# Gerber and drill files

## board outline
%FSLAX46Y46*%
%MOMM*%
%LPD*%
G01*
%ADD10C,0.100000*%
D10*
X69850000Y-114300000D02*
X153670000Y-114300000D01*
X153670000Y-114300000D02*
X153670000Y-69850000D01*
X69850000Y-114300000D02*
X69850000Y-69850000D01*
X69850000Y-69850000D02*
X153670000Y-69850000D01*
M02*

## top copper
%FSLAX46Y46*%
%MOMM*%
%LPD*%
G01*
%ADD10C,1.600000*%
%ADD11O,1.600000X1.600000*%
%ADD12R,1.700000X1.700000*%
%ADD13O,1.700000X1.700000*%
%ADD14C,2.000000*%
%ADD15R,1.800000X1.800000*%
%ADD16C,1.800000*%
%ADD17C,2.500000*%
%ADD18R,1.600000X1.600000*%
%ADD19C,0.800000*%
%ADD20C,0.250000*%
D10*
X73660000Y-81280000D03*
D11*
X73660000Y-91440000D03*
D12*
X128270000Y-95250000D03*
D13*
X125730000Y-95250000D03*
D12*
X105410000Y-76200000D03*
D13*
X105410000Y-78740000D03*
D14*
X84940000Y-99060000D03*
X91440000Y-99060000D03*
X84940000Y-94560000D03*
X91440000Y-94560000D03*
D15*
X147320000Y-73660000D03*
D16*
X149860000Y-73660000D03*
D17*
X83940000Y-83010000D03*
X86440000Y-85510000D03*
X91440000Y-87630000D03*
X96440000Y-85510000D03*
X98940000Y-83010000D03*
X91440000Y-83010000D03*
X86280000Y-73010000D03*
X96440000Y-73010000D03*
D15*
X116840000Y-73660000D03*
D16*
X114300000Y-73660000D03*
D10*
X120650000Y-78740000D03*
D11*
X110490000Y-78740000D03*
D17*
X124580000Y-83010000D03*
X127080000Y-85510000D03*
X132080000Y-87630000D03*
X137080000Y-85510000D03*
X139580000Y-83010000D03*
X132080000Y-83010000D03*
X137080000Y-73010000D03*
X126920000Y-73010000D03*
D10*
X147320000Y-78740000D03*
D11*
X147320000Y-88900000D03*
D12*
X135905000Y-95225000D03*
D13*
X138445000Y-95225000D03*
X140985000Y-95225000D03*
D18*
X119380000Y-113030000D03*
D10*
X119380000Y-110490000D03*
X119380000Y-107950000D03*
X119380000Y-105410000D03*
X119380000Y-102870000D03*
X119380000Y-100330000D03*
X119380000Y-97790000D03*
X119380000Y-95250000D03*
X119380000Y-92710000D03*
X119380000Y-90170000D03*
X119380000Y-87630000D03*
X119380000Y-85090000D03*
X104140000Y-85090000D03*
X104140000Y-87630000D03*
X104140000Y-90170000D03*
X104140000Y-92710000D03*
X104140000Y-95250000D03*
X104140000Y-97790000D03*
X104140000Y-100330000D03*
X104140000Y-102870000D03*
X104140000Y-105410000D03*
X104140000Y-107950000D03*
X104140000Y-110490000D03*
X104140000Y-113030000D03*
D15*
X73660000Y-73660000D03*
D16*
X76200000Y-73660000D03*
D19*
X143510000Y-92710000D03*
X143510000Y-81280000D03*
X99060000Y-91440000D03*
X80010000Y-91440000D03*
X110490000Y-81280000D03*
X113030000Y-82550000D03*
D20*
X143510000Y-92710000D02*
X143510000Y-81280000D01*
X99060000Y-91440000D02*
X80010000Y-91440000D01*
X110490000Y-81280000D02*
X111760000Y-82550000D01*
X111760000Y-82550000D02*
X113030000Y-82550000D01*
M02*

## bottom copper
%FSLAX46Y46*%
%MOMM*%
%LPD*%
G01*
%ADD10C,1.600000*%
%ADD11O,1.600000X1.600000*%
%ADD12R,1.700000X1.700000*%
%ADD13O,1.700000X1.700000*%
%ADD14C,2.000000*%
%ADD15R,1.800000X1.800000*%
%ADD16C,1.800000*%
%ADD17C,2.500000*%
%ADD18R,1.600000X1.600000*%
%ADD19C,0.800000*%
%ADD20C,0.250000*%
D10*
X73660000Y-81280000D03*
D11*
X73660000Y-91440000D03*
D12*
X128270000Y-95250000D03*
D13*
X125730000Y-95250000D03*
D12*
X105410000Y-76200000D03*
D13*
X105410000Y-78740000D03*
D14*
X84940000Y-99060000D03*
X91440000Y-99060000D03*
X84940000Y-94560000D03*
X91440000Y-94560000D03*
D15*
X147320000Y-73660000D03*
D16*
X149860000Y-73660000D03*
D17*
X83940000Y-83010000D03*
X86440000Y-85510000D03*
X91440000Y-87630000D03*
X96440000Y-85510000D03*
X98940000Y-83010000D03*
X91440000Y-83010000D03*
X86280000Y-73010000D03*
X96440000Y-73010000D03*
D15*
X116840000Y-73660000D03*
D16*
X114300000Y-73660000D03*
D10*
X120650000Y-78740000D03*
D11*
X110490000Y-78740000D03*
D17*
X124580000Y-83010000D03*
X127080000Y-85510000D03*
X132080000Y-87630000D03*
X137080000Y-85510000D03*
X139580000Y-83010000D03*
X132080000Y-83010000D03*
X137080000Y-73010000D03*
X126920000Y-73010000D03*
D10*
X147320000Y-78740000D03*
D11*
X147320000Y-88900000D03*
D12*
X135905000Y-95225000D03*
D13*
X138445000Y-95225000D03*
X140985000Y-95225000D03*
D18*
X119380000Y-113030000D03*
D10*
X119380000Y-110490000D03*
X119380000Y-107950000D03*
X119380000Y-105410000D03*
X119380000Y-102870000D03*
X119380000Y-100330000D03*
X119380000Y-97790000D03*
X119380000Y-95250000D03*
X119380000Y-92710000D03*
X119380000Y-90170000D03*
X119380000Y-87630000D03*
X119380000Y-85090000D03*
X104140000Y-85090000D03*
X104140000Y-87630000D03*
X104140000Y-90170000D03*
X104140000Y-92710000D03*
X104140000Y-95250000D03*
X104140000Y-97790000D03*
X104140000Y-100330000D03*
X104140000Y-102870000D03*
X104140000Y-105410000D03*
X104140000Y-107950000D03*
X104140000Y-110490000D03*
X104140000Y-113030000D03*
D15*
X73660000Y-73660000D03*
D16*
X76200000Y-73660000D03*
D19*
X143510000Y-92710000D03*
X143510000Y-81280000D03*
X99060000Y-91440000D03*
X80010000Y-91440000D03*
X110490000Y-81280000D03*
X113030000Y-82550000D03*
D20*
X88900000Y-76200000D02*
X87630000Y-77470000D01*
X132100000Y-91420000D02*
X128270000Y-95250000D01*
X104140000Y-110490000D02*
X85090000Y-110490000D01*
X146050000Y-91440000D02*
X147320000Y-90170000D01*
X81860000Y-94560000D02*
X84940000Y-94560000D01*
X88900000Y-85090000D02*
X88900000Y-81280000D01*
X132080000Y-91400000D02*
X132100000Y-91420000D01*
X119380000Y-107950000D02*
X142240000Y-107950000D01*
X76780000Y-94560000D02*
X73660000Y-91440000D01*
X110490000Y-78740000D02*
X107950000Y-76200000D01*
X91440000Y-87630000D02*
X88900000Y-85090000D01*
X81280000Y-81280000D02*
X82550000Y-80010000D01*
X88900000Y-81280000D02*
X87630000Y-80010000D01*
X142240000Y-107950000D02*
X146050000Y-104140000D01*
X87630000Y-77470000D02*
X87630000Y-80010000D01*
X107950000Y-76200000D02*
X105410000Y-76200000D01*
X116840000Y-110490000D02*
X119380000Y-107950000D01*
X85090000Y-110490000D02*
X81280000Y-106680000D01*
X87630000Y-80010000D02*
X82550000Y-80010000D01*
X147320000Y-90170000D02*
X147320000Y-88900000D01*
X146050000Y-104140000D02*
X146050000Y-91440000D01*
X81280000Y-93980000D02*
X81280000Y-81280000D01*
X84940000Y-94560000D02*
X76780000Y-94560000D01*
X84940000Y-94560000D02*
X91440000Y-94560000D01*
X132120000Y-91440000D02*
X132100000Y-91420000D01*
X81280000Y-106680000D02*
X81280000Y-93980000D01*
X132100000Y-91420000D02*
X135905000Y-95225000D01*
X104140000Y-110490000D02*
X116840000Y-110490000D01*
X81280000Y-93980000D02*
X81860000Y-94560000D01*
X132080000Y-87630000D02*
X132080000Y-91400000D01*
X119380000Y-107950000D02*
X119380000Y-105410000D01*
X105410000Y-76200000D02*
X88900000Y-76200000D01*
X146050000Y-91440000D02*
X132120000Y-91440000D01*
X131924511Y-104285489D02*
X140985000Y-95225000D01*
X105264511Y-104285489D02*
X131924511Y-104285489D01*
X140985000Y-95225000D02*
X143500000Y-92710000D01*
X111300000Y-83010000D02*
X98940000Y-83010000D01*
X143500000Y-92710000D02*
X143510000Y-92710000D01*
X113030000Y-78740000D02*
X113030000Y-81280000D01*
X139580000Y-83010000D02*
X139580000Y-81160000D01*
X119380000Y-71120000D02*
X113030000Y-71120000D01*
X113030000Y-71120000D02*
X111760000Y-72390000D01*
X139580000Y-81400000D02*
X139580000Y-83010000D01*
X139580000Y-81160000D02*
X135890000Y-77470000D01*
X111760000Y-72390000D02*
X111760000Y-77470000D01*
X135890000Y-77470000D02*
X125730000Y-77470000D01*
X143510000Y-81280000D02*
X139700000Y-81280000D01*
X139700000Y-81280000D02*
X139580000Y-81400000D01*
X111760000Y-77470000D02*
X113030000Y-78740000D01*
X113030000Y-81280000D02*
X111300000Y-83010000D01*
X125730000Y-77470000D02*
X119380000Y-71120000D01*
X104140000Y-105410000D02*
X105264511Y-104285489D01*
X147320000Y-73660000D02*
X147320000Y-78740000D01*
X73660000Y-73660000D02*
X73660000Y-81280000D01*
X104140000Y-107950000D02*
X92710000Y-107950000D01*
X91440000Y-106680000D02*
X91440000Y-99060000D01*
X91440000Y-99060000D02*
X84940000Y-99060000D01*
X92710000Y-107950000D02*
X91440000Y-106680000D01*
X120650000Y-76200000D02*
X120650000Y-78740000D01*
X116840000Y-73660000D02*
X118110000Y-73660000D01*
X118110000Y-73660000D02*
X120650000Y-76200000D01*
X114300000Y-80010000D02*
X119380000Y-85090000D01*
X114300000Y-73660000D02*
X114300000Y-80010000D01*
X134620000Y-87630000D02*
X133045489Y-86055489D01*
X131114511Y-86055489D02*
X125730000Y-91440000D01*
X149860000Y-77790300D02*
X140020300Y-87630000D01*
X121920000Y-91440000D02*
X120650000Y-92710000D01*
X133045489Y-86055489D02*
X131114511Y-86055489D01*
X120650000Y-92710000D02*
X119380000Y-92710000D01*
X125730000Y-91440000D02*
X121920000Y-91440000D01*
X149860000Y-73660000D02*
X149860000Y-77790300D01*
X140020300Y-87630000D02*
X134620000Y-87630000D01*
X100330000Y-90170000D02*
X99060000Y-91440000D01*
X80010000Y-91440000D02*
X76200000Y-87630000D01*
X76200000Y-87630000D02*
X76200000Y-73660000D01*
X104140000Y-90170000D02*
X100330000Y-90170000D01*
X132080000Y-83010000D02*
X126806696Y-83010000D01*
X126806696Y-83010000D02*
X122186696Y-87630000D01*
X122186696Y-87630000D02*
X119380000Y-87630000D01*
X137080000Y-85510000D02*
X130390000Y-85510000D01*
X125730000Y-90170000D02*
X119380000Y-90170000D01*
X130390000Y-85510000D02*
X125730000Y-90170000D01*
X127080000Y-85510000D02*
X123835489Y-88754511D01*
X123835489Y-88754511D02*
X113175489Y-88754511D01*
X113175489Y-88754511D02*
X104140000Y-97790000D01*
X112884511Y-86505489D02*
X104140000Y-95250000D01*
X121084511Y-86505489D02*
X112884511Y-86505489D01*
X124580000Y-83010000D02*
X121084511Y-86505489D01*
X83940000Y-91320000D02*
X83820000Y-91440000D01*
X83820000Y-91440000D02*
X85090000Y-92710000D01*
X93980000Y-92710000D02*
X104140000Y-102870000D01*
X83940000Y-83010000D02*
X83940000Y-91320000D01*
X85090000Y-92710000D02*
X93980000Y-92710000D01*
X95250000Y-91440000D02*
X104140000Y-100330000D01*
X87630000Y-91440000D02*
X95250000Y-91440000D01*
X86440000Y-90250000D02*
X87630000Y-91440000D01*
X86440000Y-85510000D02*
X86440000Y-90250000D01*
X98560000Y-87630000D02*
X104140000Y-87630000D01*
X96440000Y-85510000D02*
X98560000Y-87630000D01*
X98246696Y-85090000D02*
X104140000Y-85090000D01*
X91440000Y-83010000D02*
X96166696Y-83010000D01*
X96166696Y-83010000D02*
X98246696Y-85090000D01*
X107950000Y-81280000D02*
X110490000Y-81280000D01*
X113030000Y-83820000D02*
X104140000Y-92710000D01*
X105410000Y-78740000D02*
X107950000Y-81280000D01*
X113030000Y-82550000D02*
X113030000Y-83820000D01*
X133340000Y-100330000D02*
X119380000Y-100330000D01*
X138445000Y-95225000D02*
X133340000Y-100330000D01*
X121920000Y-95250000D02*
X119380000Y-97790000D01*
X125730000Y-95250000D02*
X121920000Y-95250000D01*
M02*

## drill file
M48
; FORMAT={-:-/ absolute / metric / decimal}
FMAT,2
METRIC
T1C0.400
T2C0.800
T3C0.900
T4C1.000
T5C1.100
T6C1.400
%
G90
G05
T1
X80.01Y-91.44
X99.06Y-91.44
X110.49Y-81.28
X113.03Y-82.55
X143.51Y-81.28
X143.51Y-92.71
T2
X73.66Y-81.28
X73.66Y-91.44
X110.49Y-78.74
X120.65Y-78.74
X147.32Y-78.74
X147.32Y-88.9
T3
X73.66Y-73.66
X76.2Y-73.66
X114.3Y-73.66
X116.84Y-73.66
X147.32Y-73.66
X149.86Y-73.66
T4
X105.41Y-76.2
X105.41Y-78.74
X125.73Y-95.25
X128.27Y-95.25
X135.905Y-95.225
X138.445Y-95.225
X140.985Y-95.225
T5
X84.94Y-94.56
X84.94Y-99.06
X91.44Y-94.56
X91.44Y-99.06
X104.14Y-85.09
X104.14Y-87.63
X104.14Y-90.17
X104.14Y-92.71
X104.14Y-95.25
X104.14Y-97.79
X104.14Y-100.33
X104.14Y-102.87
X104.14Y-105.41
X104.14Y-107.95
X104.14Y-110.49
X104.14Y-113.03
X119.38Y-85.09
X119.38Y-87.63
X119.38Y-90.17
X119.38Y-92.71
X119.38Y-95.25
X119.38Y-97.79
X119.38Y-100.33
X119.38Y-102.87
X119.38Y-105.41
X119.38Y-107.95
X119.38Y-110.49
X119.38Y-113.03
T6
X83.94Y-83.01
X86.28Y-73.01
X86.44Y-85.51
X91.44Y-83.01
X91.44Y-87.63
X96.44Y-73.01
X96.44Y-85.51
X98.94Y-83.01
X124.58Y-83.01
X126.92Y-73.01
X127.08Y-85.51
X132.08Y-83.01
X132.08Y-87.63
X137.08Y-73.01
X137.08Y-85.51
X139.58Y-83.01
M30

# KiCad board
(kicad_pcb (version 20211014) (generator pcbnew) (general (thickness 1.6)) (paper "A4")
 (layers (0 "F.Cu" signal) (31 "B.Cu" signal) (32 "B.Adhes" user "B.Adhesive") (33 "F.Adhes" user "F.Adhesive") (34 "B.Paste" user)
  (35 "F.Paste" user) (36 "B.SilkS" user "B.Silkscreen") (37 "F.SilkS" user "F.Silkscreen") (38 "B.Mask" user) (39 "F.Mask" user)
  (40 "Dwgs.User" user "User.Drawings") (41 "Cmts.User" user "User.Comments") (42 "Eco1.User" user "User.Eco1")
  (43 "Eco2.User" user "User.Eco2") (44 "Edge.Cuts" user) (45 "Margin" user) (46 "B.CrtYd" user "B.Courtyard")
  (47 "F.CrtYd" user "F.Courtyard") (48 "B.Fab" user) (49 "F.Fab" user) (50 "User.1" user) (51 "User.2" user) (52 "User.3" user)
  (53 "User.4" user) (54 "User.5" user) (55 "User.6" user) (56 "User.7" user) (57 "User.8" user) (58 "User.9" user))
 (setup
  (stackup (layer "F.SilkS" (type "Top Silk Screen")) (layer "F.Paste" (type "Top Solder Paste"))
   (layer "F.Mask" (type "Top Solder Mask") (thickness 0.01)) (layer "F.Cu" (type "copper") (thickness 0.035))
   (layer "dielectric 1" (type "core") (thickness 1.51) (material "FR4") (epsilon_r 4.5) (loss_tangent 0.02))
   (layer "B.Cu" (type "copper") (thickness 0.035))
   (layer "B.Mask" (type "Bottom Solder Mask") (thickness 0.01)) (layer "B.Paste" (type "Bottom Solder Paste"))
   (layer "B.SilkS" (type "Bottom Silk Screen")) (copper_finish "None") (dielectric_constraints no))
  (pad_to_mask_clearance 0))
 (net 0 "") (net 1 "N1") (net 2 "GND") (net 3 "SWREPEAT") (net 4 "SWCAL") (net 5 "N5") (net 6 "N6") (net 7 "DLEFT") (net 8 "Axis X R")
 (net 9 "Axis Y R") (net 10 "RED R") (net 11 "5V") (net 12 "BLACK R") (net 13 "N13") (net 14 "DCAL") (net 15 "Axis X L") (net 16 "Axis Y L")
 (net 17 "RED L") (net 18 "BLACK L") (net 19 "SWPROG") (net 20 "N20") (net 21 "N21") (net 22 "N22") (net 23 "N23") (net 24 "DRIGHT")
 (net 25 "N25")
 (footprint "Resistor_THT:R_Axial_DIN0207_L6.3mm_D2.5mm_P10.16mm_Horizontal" (layer "F.Cu") (at 73.66 81.28 -90)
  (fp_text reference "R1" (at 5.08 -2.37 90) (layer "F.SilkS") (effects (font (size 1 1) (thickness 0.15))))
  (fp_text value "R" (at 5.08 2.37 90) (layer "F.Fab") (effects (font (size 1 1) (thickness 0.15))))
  (pad "1" thru_hole circle (at 0 0 270) (size 1.6 1.6) (drill 0.8) (layers *.Cu *.Mask) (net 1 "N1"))
  (pad "2" thru_hole oval (at 10.16 0 270) (size 1.6 1.6) (drill 0.8) (layers *.Cu *.Mask) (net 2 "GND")))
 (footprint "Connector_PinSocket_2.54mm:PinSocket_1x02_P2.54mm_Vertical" (layer "F.Cu") (at 128.27 95.25 -90)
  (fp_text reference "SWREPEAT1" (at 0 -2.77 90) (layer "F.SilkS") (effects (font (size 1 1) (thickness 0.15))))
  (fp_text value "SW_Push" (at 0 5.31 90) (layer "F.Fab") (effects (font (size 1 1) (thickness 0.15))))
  (pad "1" thru_hole rect (at 0 0 270) (size 1.7 1.7) (drill 1) (layers *.Cu *.Mask) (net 2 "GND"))
  (pad "2" thru_hole oval (at 0 2.54 270) (size 1.7 1.7) (drill 1) (layers *.Cu *.Mask) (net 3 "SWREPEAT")))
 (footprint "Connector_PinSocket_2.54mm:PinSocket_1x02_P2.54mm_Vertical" (layer "F.Cu") (at 105.41 76.2)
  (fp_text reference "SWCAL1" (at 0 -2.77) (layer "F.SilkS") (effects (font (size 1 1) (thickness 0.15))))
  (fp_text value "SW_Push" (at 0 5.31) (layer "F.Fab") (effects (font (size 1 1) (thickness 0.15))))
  (pad "1" thru_hole rect (at 0 0) (size 1.7 1.7) (drill 1) (layers *.Cu *.Mask) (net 2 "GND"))
  (pad "2" thru_hole oval (at 0 2.54) (size 1.7 1.7) (drill 1) (layers *.Cu *.Mask) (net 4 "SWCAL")))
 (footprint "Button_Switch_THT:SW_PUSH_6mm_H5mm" (layer "F.Cu") (at 91.44 99.06 180)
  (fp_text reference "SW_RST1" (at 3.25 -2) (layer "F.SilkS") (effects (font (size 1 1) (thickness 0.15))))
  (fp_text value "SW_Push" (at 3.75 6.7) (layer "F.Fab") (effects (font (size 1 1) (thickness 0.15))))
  (pad "1" thru_hole circle (at 6.5 0 270) (size 2 2) (drill 1.1) (layers *.Cu *.Mask) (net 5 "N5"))
  (pad "1" thru_hole circle (at 0 0 270) (size 2 2) (drill 1.1) (layers *.Cu *.Mask) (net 5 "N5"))
  (pad "2" thru_hole circle (at 6.5 4.5 270) (size 2 2) (drill 1.1) (layers *.Cu *.Mask) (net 2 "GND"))
  (pad "2" thru_hole circle (at 0 4.5 270) (size 2 2) (drill 1.1) (layers *.Cu *.Mask) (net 2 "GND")))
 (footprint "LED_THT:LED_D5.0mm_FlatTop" (layer "F.Cu") (at 147.32 73.66)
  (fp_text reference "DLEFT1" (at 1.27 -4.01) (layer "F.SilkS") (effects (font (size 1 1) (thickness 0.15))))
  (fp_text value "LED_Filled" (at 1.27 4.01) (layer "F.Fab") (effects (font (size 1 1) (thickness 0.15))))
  (pad "1" thru_hole rect (at 0 0) (size 1.8 1.8) (drill 0.9) (layers *.Cu *.Mask) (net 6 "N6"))
  (pad "2" thru_hole circle (at 2.54 0) (size 1.8 1.8) (drill 0.9) (layers *.Cu *.Mask) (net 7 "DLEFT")))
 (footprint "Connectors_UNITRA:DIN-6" (layer "F.Cu") (at 91.44 80.01 180)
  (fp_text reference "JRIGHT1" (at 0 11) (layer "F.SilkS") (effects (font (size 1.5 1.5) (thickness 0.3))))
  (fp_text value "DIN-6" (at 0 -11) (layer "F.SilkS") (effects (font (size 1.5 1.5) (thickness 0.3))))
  (pad "1" thru_hole circle locked (at 7.5 -3 180) (size 2.5 2.5) (drill 1.4) (layers *.Cu *.Mask) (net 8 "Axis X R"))
  (pad "2" thru_hole circle locked (at 5 -5.5 180) (size 2.5 2.5) (drill 1.4) (layers *.Cu *.Mask) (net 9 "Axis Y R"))
  (pad "3" thru_hole circle locked (at 0 -7.62 180) (size 2.5 2.5) (drill 1.4) (layers *.Cu *.Mask) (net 2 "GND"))
  (pad "4" thru_hole circle locked (at -5 -5.5 180) (size 2.5 2.5) (drill 1.4) (layers *.Cu *.Mask) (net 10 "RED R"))
  (pad "5" thru_hole circle locked (at -7.5 -3 180) (size 2.5 2.5) (drill 1.4) (layers *.Cu *.Mask) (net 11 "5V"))
  (pad "6" thru_hole circle locked (at 0 -3 180) (size 2.5 2.5) (drill 1.4) (layers *.Cu *.Mask) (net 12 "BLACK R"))
  (pad "7" thru_hole circle locked (at 5.16 7 180) (size 2.5 2.5) (drill 1.4) (layers *.Cu *.Mask))
  (pad "7" thru_hole circle locked (at -5 7 180) (size 2.5 2.5) (drill 1.4) (layers *.Cu *.Mask)))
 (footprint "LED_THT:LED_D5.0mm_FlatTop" (layer "F.Cu") (at 116.84 73.66 180)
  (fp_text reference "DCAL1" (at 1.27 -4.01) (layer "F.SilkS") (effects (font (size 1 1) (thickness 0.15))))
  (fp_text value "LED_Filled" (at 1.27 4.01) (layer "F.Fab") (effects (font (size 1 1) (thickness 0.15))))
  (pad "1" thru_hole rect (at 0 0 180) (size 1.8 1.8) (drill 0.9) (layers *.Cu *.Mask) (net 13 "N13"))
  (pad "2" thru_hole circle (at 2.54 0 180) (size 1.8 1.8) (drill 0.9) (layers *.Cu *.Mask) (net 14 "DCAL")))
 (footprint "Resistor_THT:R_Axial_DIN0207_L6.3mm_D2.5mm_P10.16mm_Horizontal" (layer "F.Cu") (at 120.65 78.74 180)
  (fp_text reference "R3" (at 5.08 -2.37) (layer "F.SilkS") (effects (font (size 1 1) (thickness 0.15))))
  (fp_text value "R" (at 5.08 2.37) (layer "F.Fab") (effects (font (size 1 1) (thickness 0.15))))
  (pad "1" thru_hole circle (at 0 0 180) (size 1.6 1.6) (drill 0.8) (layers *.Cu *.Mask) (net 13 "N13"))
  (pad "2" thru_hole oval (at 10.16 0 180) (size 1.6 1.6) (drill 0.8) (layers *.Cu *.Mask) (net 2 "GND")))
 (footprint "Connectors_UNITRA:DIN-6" (layer "F.Cu") (at 132.08 80.01 180)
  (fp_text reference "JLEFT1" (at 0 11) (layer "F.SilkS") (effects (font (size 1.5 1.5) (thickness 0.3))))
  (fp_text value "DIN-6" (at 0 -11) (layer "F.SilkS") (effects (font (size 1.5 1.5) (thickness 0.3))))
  (pad "1" thru_hole circle locked (at 7.5 -3 180) (size 2.5 2.5) (drill 1.4) (layers *.Cu *.Mask) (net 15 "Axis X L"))
  (pad "2" thru_hole circle locked (at 5 -5.5 180) (size 2.5 2.5) (drill 1.4) (layers *.Cu *.Mask) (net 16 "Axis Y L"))
  (pad "3" thru_hole circle locked (at 0 -7.62 180) (size 2.5 2.5) (drill 1.4) (layers *.Cu *.Mask) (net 2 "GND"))
  (pad "4" thru_hole circle locked (at -5 -5.5 180) (size 2.5 2.5) (drill 1.4) (layers *.Cu *.Mask) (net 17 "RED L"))
  (pad "5" thru_hole circle locked (at -7.5 -3 180) (size 2.5 2.5) (drill 1.4) (layers *.Cu *.Mask) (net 11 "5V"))
  (pad "6" thru_hole circle locked (at 0 -3 180) (size 2.5 2.5) (drill 1.4) (layers *.Cu *.Mask) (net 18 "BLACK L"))
  (pad "7" thru_hole circle locked (at -5 7 180) (size 2.5 2.5) (drill 1.4) (layers *.Cu *.Mask))
  (pad "7" thru_hole circle locked (at 5.16 7 180) (size 2.5 2.5) (drill 1.4) (layers *.Cu *.Mask)))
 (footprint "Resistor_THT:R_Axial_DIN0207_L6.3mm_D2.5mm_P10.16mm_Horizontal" (layer "F.Cu") (at 147.32 78.74 -90)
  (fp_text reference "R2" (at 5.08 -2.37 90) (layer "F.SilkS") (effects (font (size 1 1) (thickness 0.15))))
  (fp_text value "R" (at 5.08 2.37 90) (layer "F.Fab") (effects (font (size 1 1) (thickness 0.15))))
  (pad "1" thru_hole circle (at 0 0 270) (size 1.6 1.6) (drill 0.8) (layers *.Cu *.Mask) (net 6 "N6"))
  (pad "2" thru_hole oval (at 10.16 0 270) (size 1.6 1.6) (drill 0.8) (layers *.Cu *.Mask) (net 2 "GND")))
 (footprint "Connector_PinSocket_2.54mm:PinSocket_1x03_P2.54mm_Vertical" (layer "F.Cu") (at 135.905 95.225 90)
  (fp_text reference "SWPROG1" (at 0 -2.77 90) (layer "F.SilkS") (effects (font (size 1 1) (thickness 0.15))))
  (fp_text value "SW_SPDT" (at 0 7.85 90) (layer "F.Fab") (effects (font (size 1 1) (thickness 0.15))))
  (pad "1" thru_hole rect (at 0 0 90) (size 1.7 1.7) (drill 1) (layers *.Cu *.Mask) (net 2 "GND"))
  (pad "2" thru_hole oval (at 0 2.54 90) (size 1.7 1.7) (drill 1) (layers *.Cu *.Mask) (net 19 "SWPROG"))
  (pad "3" thru_hole oval (at 0 5.08 90) (size 1.7 1.7) (drill 1) (layers *.Cu *.Mask) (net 11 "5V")))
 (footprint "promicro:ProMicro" (layer "F.Cu") (at 111.76 99.06 90)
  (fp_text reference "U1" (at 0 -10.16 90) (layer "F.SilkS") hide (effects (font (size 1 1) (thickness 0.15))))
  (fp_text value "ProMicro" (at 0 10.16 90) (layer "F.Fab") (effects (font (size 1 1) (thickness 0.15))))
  (pad "1" thru_hole rect locked (at -13.97 7.62 90) (size 1.6 1.6) (drill 1.1) (layers *.Cu *.Mask "F.SilkS") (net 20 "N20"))
  (pad "2" thru_hole circle locked (at -11.43 7.62 90) (size 1.6 1.6) (drill 1.1) (layers *.Cu *.Mask "F.SilkS") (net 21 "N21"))
  (pad "3" thru_hole circle locked (at -8.89 7.62 90) (size 1.6 1.6) (drill 1.1) (layers *.Cu *.Mask "F.SilkS") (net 2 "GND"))
  (pad "4" thru_hole circle locked (at -6.35 7.62 90) (size 1.6 1.6) (drill 1.1) (layers *.Cu *.Mask "F.SilkS") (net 2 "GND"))
  (pad "5" thru_hole circle locked (at -3.81 7.62 90) (size 1.6 1.6) (drill 1.1) (layers *.Cu *.Mask "F.SilkS") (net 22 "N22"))
  (pad "6" thru_hole circle locked (at -1.27 7.62 90) (size 1.6 1.6) (drill 1.1) (layers *.Cu *.Mask "F.SilkS") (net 19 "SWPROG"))
  (pad "7" thru_hole circle locked (at 1.27 7.62 90) (size 1.6 1.6) (drill 1.1) (layers *.Cu *.Mask "F.SilkS") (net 3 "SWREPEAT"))
  (pad "8" thru_hole circle locked (at 3.81 7.62 90) (size 1.6 1.6) (drill 1.1) (layers *.Cu *.Mask "F.SilkS") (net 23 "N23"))
  (pad "9" thru_hole circle locked (at 6.35 7.62 90) (size 1.6 1.6) (drill 1.1) (layers *.Cu *.Mask "F.SilkS") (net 7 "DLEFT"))
  (pad "10" thru_hole circle locked (at 8.89 7.62 90) (size 1.6 1.6) (drill 1.1) (layers *.Cu *.Mask "F.SilkS") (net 17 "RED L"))
  (pad "11" thru_hole circle locked (at 11.43 7.62 90) (size 1.6 1.6) (drill 1.1) (layers *.Cu *.Mask "F.SilkS") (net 18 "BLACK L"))
  (pad "12" thru_hole circle locked (at 13.97 7.62 90) (size 1.6 1.6) (drill 1.1) (layers *.Cu *.Mask "F.SilkS") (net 14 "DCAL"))
  (pad "13" thru_hole circle locked (at 13.97 -7.62 90) (size 1.6 1.6) (drill 1.1) (layers *.Cu *.Mask "F.SilkS") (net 12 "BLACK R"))
  (pad "14" thru_hole circle locked (at 11.43 -7.62 90) (size 1.6 1.6) (drill 1.1) (layers *.Cu *.Mask "F.SilkS") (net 10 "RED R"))
  (pad "15" thru_hole circle locked (at 8.89 -7.62 90) (size 1.6 1.6) (drill 1.1) (layers *.Cu *.Mask "F.SilkS") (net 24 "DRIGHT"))
  (pad "16" thru_hole circle locked (at 6.35 -7.62 90) (size 1.6 1.6) (drill 1.1) (layers *.Cu *.Mask "F.SilkS") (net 4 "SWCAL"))
  (pad "17" thru_hole circle locked (at 3.81 -7.62 90) (size 1.6 1.6) (drill 1.1) (layers *.Cu *.Mask "F.SilkS") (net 15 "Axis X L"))
  (pad "18" thru_hole circle locked (at 1.27 -7.62 90) (size 1.6 1.6) (drill 1.1) (layers *.Cu *.Mask "F.SilkS") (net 16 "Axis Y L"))
  (pad "19" thru_hole circle locked (at -1.27 -7.62 90) (size 1.6 1.6) (drill 1.1) (layers *.Cu *.Mask "F.SilkS") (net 9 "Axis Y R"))
  (pad "20" thru_hole circle locked (at -3.81 -7.62 90) (size 1.6 1.6) (drill 1.1) (layers *.Cu *.Mask "F.SilkS") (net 8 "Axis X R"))
  (pad "21" thru_hole circle locked (at -6.35 -7.62 90) (size 1.6 1.6) (drill 1.1) (layers *.Cu *.Mask "F.SilkS") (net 11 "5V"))
  (pad "22" thru_hole circle locked (at -8.89 -7.62 90) (size 1.6 1.6) (drill 1.1) (layers *.Cu *.Mask "F.SilkS") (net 5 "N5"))
  (pad "23" thru_hole circle locked (at -11.43 -7.62 90) (size 1.6 1.6) (drill 1.1) (layers *.Cu *.Mask "F.SilkS") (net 2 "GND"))
  (pad "24" thru_hole circle locked (at -13.97 -7.62 90) (size 1.6 1.6) (drill 1.1) (layers *.Cu *.Mask "F.SilkS") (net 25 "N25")))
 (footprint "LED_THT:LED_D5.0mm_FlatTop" (layer "F.Cu") (at 73.66 73.66)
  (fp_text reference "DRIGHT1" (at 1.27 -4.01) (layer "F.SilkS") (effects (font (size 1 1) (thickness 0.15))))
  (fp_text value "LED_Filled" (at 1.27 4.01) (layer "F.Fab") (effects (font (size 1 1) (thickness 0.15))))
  (pad "1" thru_hole rect (at 0 0) (size 1.8 1.8) (drill 0.9) (layers *.Cu *.Mask) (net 1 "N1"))
  (pad "2" thru_hole circle (at 2.54 0) (size 1.8 1.8) (drill 0.9) (layers *.Cu *.Mask) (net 24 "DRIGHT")))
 (gr_line (start 69.85 114.3) (end 153.67 114.3) (layer "Edge.Cuts") (width 0.1))
 (gr_line (start 153.67 114.3) (end 153.67 69.85) (layer "Edge.Cuts") (width 0.1))
 (gr_line (start 69.85 114.3) (end 69.85 69.85) (layer "Edge.Cuts") (width 0.1))
 (gr_line (start 69.85 69.85) (end 153.67 69.85) (layer "Edge.Cuts") (width 0.1))
 (segment (start 88.9 76.2) (end 87.63 77.47) (width 0.25) (layer "B.Cu") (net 2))
 (segment (start 132.1 91.42) (end 128.27 95.25) (width 0.25) (layer "B.Cu") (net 2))
 (segment (start 104.14 110.49) (end 85.09 110.49) (width 0.25) (layer "B.Cu") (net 2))
 (segment (start 146.05 91.44) (end 147.32 90.17) (width 0.25) (layer "B.Cu") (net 2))
 (segment (start 81.86 94.56) (end 84.94 94.56) (width 0.25) (layer "B.Cu") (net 2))
 (segment (start 88.9 85.09) (end 88.9 81.28) (width 0.25) (layer "B.Cu") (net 2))
 (segment (start 132.08 91.4) (end 132.1 91.42) (width 0.25) (layer "B.Cu") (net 2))
 (segment (start 119.38 107.95) (end 142.24 107.95) (width 0.25) (layer "B.Cu") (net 2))
 (segment (start 76.78 94.56) (end 73.66 91.44) (width 0.25) (layer "B.Cu") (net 2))
 (segment (start 110.49 78.74) (end 107.95 76.2) (width 0.25) (layer "B.Cu") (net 2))
 (segment (start 91.44 87.63) (end 88.9 85.09) (width 0.25) (layer "B.Cu") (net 2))
 (segment (start 81.28 81.28) (end 82.55 80.01) (width 0.25) (layer "B.Cu") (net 2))
 (segment (start 88.9 81.28) (end 87.63 80.01) (width 0.25) (layer "B.Cu") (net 2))
 (segment (start 142.24 107.95) (end 146.05 104.14) (width 0.25) (layer "B.Cu") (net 2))
 (segment (start 87.63 77.47) (end 87.63 80.01) (width 0.25) (layer "B.Cu") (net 2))
 (segment (start 107.95 76.2) (end 105.41 76.2) (width 0.25) (layer "B.Cu") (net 2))
 (segment (start 116.84 110.49) (end 119.38 107.95) (width 0.25) (layer "B.Cu") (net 2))
 (segment (start 85.09 110.49) (end 81.28 106.68) (width 0.25) (layer "B.Cu") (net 2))
 (segment (start 87.63 80.01) (end 82.55 80.01) (width 0.25) (layer "B.Cu") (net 2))
 (segment (start 147.32 90.17) (end 147.32 88.9) (width 0.25) (layer "B.Cu") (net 2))
 (segment (start 146.05 104.14) (end 146.05 91.44) (width 0.25) (layer "B.Cu") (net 2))
 (segment (start 81.28 93.98) (end 81.28 81.28) (width 0.25) (layer "B.Cu") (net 2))
 (segment (start 84.94 94.56) (end 76.78 94.56) (width 0.25) (layer "B.Cu") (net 2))
 (segment (start 84.94 94.56) (end 91.44 94.56) (width 0.25) (layer "B.Cu") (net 2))
 (segment (start 132.12 91.44) (end 132.1 91.42) (width 0.25) (layer "B.Cu") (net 2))
 (segment (start 81.28 106.68) (end 81.28 93.98) (width 0.25) (layer "B.Cu") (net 2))
 (segment (start 132.1 91.42) (end 135.905 95.225) (width 0.25) (layer "B.Cu") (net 2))
 (segment (start 104.14 110.49) (end 116.84 110.49) (width 0.25) (layer "B.Cu") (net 2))
 (segment (start 81.28 93.98) (end 81.86 94.56) (width 0.25) (layer "B.Cu") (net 2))
 (segment (start 132.08 87.63) (end 132.08 91.4) (width 0.25) (layer "B.Cu") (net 2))
 (segment (start 119.38 107.95) (end 119.38 105.41) (width 0.25) (layer "B.Cu") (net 2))
 (segment (start 105.41 76.2) (end 88.9 76.2) (width 0.25) (layer "B.Cu") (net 2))
 (segment (start 146.05 91.44) (end 132.12 91.44) (width 0.25) (layer "B.Cu") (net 2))
 (segment (start 143.51 92.71) (end 143.51 81.28) (width 0.25) (layer "F.Cu") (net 11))
 (via (at 143.51 92.71) (size 0.8) (drill 0.4) (layers "F.Cu" "B.Cu") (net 11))
 (via (at 143.51 81.28) (size 0.8) (drill 0.4) (layers "F.Cu" "B.Cu") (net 11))
 (segment (start 131.924511 104.285489) (end 140.985 95.225) (width 0.25) (layer "B.Cu") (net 11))
 (segment (start 105.264511 104.285489) (end 131.924511 104.285489) (width 0.25) (layer "B.Cu") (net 11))
 (segment (start 140.985 95.225) (end 143.5 92.71) (width 0.25) (layer "B.Cu") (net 11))
 (segment (start 111.3 83.01) (end 98.94 83.01) (width 0.25) (layer "B.Cu") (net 11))
 (segment (start 143.5 92.71) (end 143.51 92.71) (width 0.25) (layer "B.Cu") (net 11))
 (segment (start 113.03 78.74) (end 113.03 81.28) (width 0.25) (layer "B.Cu") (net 11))
 (segment (start 139.58 83.01) (end 139.58 81.16) (width 0.25) (layer "B.Cu") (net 11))
 (segment (start 119.38 71.12) (end 113.03 71.12) (width 0.25) (layer "B.Cu") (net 11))
 (segment (start 113.03 71.12) (end 111.76 72.39) (width 0.25) (layer "B.Cu") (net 11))
 (segment (start 139.58 81.4) (end 139.58 83.01) (width 0.25) (layer "B.Cu") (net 11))
 (segment (start 139.58 81.16) (end 135.89 77.47) (width 0.25) (layer "B.Cu") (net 11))
 (segment (start 111.76 72.39) (end 111.76 77.47) (width 0.25) (layer "B.Cu") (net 11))
 (segment (start 135.89 77.47) (end 125.73 77.47) (width 0.25) (layer "B.Cu") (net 11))
 (segment (start 143.51 81.28) (end 139.7 81.28) (width 0.25) (layer "B.Cu") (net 11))
 (segment (start 139.7 81.28) (end 139.58 81.4) (width 0.25) (layer "B.Cu") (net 11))
 (segment (start 111.76 77.47) (end 113.03 78.74) (width 0.25) (layer "B.Cu") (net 11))
 (segment (start 113.03 81.28) (end 111.3 83.01) (width 0.25) (layer "B.Cu") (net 11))
 (segment (start 125.73 77.47) (end 119.38 71.12) (width 0.25) (layer "B.Cu") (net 11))
 (segment (start 104.14 105.41) (end 105.264511 104.285489) (width 0.25) (layer "B.Cu") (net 11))
 (segment (start 147.32 73.66) (end 147.32 78.74) (width 0.25) (layer "B.Cu") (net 6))
 (segment (start 73.66 73.66) (end 73.66 81.28) (width 0.25) (layer "B.Cu") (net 1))
 (segment (start 104.14 107.95) (end 92.71 107.95) (width 0.25) (layer "B.Cu") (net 5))
 (segment (start 91.44 106.68) (end 91.44 99.06) (width 0.25) (layer "B.Cu") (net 5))
 (segment (start 91.44 99.06) (end 84.94 99.06) (width 0.25) (layer "B.Cu") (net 5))
 (segment (start 92.71 107.95) (end 91.44 106.68) (width 0.25) (layer "B.Cu") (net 5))
 (segment (start 120.65 76.2) (end 120.65 78.74) (width 0.25) (layer "B.Cu") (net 13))
 (segment (start 116.84 73.66) (end 118.11 73.66) (width 0.25) (layer "B.Cu") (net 13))
 (segment (start 118.11 73.66) (end 120.65 76.2) (width 0.25) (layer "B.Cu") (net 13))
 (segment (start 114.3 80.01) (end 119.38 85.09) (width 0.25) (layer "B.Cu") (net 14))
 (segment (start 114.3 73.66) (end 114.3 80.01) (width 0.25) (layer "B.Cu") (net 14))
 (segment (start 134.62 87.63) (end 133.045489 86.055489) (width 0.25) (layer "B.Cu") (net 7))
 (segment (start 131.114511 86.055489) (end 125.73 91.44) (width 0.25) (layer "B.Cu") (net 7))
 (segment (start 149.86 77.7903) (end 140.0203 87.63) (width 0.25) (layer "B.Cu") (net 7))
 (segment (start 121.92 91.44) (end 120.65 92.71) (width 0.25) (layer "B.Cu") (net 7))
 (segment (start 133.045489 86.055489) (end 131.114511 86.055489) (width 0.25) (layer "B.Cu") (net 7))
 (segment (start 120.65 92.71) (end 119.38 92.71) (width 0.25) (layer "B.Cu") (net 7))
 (segment (start 125.73 91.44) (end 121.92 91.44) (width 0.25) (layer "B.Cu") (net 7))
 (segment (start 149.86 73.66) (end 149.86 77.7903) (width 0.25) (layer "B.Cu") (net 7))
 (segment (start 140.0203 87.63) (end 134.62 87.63) (width 0.25) (layer "B.Cu") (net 7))
 (segment (start 99.06 91.44) (end 80.01 91.44) (width 0.25) (layer "F.Cu") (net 24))
 (via (at 99.06 91.44) (size 0.8) (drill 0.4) (layers "F.Cu" "B.Cu") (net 24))
 (via (at 80.01 91.44) (size 0.8) (drill 0.4) (layers "F.Cu" "B.Cu") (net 24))
 (segment (start 100.33 90.17) (end 99.06 91.44) (width 0.25) (layer "B.Cu") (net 24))
 (segment (start 80.01 91.44) (end 76.2 87.63) (width 0.25) (layer "B.Cu") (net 24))
 (segment (start 76.2 87.63) (end 76.2 73.66) (width 0.25) (layer "B.Cu") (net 24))
 (segment (start 104.14 90.17) (end 100.33 90.17) (width 0.25) (layer "B.Cu") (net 24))
 (segment (start 132.08 83.01) (end 126.806696 83.01) (width 0.25) (layer "B.Cu") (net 18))
 (segment (start 126.806696 83.01) (end 122.186696 87.63) (width 0.25) (layer "B.Cu") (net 18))
 (segment (start 122.186696 87.63) (end 119.38 87.63) (width 0.25) (layer "B.Cu") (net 18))
 (segment (start 137.08 85.51) (end 130.39 85.51) (width 0.25) (layer "B.Cu") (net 17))
 (segment (start 125.73 90.17) (end 119.38 90.17) (width 0.25) (layer "B.Cu") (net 17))
 (segment (start 130.39 85.51) (end 125.73 90.17) (width 0.25) (layer "B.Cu") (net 17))
 (segment (start 127.08 85.51) (end 123.835489 88.754511) (width 0.25) (layer "B.Cu") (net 16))
 (segment (start 123.835489 88.754511) (end 113.175489 88.754511) (width 0.25) (layer "B.Cu") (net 16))
 (segment (start 113.175489 88.754511) (end 104.14 97.79) (width 0.25) (layer "B.Cu") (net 16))
 (segment (start 112.884511 86.505489) (end 104.14 95.25) (width 0.25) (layer "B.Cu") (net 15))
 (segment (start 121.084511 86.505489) (end 112.884511 86.505489) (width 0.25) (layer "B.Cu") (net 15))
 (segment (start 124.58 83.01) (end 121.084511 86.505489) (width 0.25) (layer "B.Cu") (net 15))
 (segment (start 83.94 91.32) (end 83.82 91.44) (width 0.25) (layer "B.Cu") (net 8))
 (segment (start 83.82 91.44) (end 85.09 92.71) (width 0.25) (layer "B.Cu") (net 8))
 (segment (start 93.98 92.71) (end 104.14 102.87) (width 0.25) (layer "B.Cu") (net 8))
 (segment (start 83.94 83.01) (end 83.94 91.32) (width 0.25) (layer "B.Cu") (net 8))
 (segment (start 85.09 92.71) (end 93.98 92.71) (width 0.25) (layer "B.Cu") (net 8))
 (segment (start 95.25 91.44) (end 104.14 100.33) (width 0.25) (layer "B.Cu") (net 9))
 (segment (start 87.63 91.44) (end 95.25 91.44) (width 0.25) (layer "B.Cu") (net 9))
 (segment (start 86.44 90.25) (end 87.63 91.44) (width 0.25) (layer "B.Cu") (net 9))
 (segment (start 86.44 85.51) (end 86.44 90.25) (width 0.25) (layer "B.Cu") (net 9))
 (segment (start 98.56 87.63) (end 104.14 87.63) (width 0.25) (layer "B.Cu") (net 10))
 (segment (start 96.44 85.51) (end 98.56 87.63) (width 0.25) (layer "B.Cu") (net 10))
 (segment (start 98.246696 85.09) (end 104.14 85.09) (width 0.25) (layer "B.Cu") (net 12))
 (segment (start 91.44 83.01) (end 96.166696 83.01) (width 0.25) (layer "B.Cu") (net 12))
 (segment (start 96.166696 83.01) (end 98.246696 85.09) (width 0.25) (layer "B.Cu") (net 12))
 (segment (start 110.49 81.28) (end 111.76 82.55) (width 0.25) (layer "F.Cu") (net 4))
 (segment (start 111.76 82.55) (end 113.03 82.55) (width 0.25) (layer "F.Cu") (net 4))
 (via (at 110.49 81.28) (size 0.8) (drill 0.4) (layers "F.Cu" "B.Cu") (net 4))
 (via (at 113.03 82.55) (size 0.8) (drill 0.4) (layers "F.Cu" "B.Cu") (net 4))
 (segment (start 107.95 81.28) (end 110.49 81.28) (width 0.25) (layer "B.Cu") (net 4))
 (segment (start 113.03 83.82) (end 104.14 92.71) (width 0.25) (layer "B.Cu") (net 4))
 (segment (start 105.41 78.74) (end 107.95 81.28) (width 0.25) (layer "B.Cu") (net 4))
 (segment (start 113.03 82.55) (end 113.03 83.82) (width 0.25) (layer "B.Cu") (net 4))
 (segment (start 133.34 100.33) (end 119.38 100.33) (width 0.25) (layer "B.Cu") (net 19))
 (segment (start 138.445 95.225) (end 133.34 100.33) (width 0.25) (layer "B.Cu") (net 19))
 (segment (start 121.92 95.25) (end 119.38 97.79) (width 0.25) (layer "B.Cu") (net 3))
 (segment (start 125.73 95.25) (end 121.92 95.25) (width 0.25) (layer "B.Cu") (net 3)))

